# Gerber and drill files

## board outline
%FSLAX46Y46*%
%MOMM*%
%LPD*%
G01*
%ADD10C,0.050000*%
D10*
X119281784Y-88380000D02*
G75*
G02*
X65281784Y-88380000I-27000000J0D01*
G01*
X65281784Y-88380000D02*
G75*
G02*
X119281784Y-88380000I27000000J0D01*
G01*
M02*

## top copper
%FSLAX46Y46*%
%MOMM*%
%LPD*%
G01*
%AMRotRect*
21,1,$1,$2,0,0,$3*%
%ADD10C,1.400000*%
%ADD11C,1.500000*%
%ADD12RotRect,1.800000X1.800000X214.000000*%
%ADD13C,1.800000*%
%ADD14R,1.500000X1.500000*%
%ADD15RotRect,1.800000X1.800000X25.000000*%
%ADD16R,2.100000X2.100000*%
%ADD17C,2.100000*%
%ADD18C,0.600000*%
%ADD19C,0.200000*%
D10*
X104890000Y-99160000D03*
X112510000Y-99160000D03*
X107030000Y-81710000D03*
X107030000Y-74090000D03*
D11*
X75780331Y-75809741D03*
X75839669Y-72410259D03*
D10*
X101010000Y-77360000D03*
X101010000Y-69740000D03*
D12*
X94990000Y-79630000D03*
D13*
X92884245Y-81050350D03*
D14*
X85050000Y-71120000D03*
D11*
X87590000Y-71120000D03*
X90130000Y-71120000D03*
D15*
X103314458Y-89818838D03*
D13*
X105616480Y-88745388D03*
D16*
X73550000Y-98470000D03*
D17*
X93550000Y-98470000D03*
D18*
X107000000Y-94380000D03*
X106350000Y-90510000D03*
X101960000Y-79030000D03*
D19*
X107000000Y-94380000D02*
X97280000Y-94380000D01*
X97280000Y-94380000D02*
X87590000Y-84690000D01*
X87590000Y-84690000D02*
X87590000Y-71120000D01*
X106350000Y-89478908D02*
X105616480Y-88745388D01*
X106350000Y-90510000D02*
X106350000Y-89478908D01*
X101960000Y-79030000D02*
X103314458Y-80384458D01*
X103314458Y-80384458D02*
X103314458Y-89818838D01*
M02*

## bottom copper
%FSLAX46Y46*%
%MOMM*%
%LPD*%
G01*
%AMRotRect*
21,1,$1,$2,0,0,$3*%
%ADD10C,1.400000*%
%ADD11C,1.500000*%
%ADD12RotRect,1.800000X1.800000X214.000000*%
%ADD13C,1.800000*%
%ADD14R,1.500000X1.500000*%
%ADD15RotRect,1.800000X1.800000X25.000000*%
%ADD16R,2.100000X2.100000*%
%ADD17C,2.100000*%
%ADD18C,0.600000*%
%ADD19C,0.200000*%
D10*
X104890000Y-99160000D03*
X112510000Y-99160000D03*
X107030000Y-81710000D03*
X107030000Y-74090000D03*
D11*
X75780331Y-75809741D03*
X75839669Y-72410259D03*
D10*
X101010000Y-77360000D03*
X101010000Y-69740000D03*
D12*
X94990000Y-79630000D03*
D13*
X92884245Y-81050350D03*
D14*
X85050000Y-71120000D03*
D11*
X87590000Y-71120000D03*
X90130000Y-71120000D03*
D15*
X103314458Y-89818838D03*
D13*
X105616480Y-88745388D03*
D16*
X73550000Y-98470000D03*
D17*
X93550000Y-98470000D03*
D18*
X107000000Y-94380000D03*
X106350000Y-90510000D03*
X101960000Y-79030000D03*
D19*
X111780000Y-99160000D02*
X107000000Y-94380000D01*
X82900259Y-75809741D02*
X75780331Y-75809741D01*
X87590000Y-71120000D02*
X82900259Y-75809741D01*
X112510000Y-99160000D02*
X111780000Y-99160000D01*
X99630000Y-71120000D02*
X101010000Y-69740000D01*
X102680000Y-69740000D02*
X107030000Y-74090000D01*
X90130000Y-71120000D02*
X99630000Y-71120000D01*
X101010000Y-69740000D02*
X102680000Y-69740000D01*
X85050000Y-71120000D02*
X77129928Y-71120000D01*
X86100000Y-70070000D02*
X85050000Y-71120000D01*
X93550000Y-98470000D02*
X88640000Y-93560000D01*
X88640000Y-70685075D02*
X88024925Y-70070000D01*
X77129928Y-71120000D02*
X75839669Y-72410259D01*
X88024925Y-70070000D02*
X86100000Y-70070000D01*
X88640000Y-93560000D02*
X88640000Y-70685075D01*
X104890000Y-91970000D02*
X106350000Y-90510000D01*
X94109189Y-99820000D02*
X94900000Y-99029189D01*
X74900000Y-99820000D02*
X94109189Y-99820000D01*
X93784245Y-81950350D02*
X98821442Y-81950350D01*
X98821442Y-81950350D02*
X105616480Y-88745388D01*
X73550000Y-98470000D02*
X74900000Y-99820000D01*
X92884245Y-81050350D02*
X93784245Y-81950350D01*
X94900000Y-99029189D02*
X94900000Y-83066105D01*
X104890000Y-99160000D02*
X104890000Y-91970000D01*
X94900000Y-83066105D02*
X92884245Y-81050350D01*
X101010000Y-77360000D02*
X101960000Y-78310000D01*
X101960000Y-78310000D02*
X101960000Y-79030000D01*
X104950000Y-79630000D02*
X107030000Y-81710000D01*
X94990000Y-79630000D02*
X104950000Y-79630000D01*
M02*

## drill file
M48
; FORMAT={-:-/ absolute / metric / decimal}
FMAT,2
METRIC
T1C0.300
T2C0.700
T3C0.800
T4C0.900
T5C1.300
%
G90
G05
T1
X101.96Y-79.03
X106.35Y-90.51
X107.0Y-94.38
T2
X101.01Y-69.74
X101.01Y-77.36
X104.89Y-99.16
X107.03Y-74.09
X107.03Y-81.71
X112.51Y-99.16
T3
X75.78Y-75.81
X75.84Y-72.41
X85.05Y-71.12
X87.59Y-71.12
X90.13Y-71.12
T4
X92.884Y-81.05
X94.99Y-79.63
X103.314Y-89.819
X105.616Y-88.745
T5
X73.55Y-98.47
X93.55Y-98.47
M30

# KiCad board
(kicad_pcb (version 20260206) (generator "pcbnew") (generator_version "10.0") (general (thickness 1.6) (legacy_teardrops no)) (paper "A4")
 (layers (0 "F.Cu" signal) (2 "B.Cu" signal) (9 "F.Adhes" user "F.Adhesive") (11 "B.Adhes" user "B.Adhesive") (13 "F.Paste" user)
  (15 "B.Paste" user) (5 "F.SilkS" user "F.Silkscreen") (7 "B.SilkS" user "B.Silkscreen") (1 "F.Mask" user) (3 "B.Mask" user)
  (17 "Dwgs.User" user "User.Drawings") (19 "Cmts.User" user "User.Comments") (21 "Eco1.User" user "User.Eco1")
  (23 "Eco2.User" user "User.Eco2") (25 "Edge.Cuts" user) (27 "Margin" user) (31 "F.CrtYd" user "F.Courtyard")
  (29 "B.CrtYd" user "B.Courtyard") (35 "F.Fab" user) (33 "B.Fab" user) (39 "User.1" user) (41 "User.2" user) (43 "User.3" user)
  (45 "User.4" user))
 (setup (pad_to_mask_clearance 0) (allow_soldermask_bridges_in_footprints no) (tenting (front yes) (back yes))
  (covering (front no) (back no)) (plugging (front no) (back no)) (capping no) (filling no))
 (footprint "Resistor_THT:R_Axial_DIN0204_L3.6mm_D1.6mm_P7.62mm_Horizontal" (layer "F.Cu") (at 104.89 99.16)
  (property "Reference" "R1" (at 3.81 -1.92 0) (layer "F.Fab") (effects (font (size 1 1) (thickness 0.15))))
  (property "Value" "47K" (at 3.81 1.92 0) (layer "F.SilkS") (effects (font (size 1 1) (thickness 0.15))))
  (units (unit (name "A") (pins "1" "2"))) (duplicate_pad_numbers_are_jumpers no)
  (pad "1" thru_hole circle (at 0 0) (size 1.4 1.4) (drill 0.7) (layers "*.Cu" "*.Mask") (remove_unused_layers no) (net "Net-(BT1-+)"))
  (pad "2" thru_hole circle (at 7.62 0) (size 1.4 1.4) (drill 0.7) (layers "*.Cu" "*.Mask") (remove_unused_layers no) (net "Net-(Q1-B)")))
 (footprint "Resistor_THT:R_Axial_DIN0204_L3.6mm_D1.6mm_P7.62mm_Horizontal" (layer "F.Cu") (at 107.03 81.71 90)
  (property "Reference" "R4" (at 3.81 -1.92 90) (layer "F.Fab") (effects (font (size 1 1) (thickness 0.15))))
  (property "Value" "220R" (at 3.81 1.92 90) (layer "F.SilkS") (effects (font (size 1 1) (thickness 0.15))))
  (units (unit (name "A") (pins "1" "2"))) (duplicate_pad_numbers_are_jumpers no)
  (pad "1" thru_hole circle (at 0 0 90) (size 1.4 1.4) (drill 0.7) (layers "*.Cu" "*.Mask") (remove_unused_layers no) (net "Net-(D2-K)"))
  (pad "2" thru_hole circle (at 7.62 0 90) (size 1.4 1.4) (drill 0.7) (layers "*.Cu" "*.Mask") (remove_unused_layers no) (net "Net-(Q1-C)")))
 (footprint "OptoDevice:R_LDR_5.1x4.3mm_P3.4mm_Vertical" (layer "F.Cu") (at 75.780331 75.809741 89)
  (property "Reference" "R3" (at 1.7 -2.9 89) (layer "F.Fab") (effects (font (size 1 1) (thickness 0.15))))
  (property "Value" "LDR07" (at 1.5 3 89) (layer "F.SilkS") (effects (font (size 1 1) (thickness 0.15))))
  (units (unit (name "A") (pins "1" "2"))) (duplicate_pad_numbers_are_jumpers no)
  (pad "1" thru_hole circle (at 0 0 89) (size 1.5 1.5) (drill 0.8) (layers "*.Cu" "*.Mask") (remove_unused_layers no) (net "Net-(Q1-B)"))
  (pad "2" thru_hole circle (at 3.4 0 89) (size 1.5 1.5) (drill 0.8) (layers "*.Cu" "*.Mask") (remove_unused_layers no) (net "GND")))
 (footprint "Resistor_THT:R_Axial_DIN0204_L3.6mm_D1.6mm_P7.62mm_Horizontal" (layer "F.Cu") (at 101.01 77.36 90)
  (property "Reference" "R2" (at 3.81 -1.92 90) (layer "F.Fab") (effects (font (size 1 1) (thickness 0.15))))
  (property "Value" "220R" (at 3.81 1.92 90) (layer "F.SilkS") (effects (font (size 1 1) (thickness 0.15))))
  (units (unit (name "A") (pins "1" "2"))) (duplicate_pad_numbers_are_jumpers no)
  (pad "1" thru_hole circle (at 0 0 90) (size 1.4 1.4) (drill 0.7) (layers "*.Cu" "*.Mask") (remove_unused_layers no) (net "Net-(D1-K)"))
  (pad "2" thru_hole circle (at 7.62 0 90) (size 1.4 1.4) (drill 0.7) (layers "*.Cu" "*.Mask") (remove_unused_layers no) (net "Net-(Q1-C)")))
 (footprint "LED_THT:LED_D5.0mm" (layer "F.Cu") (at 94.99 79.63 -146)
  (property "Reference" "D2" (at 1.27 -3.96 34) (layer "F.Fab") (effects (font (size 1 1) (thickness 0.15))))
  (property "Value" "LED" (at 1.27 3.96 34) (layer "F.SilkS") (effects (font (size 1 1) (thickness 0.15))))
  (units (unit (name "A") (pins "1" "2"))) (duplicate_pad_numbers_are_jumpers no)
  (pad "1" thru_hole rect (at 0 0 214) (size 1.8 1.8) (drill 0.9) (layers "*.Cu" "*.Mask") (remove_unused_layers no) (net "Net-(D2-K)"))
  (pad "2" thru_hole circle (at 2.54 0 214) (size 1.8 1.8) (drill 0.9) (layers "*.Cu" "*.Mask") (remove_unused_layers no)
   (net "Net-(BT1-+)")))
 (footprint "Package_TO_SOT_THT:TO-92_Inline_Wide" (layer "F.Cu") (at 85.05 71.12)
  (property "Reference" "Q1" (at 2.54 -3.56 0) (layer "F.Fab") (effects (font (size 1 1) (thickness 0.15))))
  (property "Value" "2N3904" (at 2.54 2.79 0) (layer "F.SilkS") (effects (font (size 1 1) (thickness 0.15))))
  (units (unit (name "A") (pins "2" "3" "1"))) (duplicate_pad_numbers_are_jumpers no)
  (pad "1" thru_hole rect (at 0 0) (size 1.5 1.5) (drill 0.8) (layers "*.Cu" "*.Mask") (remove_unused_layers no) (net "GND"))
  (pad "2" thru_hole circle (at 2.54 0) (size 1.5 1.5) (drill 0.8) (layers "*.Cu" "*.Mask") (remove_unused_layers no) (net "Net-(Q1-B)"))
  (pad "3" thru_hole circle (at 5.08 0) (size 1.5 1.5) (drill 0.8) (layers "*.Cu" "*.Mask") (remove_unused_layers no) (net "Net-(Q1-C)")))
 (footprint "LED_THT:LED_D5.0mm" (layer "F.Cu") (at 103.314458 89.818838 25)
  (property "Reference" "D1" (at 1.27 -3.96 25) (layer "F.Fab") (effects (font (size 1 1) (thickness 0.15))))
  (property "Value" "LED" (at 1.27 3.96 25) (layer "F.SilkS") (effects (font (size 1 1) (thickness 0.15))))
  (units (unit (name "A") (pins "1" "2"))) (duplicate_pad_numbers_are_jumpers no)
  (pad "1" thru_hole rect (at 0 0 25) (size 1.8 1.8) (drill 0.9) (layers "*.Cu" "*.Mask") (remove_unused_layers no) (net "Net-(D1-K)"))
  (pad "2" thru_hole circle (at 2.54 0 25) (size 1.8 1.8) (drill 0.9) (layers "*.Cu" "*.Mask") (remove_unused_layers no) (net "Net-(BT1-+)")))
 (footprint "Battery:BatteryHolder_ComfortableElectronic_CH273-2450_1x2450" (layer "B.Cu") (at 73.55 98.47)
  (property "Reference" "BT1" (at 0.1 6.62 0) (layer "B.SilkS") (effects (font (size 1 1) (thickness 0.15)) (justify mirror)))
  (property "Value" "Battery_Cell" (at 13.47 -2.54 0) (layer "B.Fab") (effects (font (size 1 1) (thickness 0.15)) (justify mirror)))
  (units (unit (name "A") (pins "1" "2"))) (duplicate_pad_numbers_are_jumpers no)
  (pad "1" thru_hole rect (at 0 0 90) (size 2.1 2.1) (drill 1.3) (layers "*.Cu" "*.Mask") (remove_unused_layers no) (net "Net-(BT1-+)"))
  (pad "2" thru_hole circle (at 20 0 90) (size 2.1 2.1) (drill 1.3) (layers "*.Cu" "*.Mask") (remove_unused_layers no) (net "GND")))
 (gr_circle (center 92.281784 88.38) (end 119.281784 88.38) (stroke (width 0.05) (type solid)) (fill no) (layer "Edge.Cuts"))
 (segment (start 107 94.38) (end 97.28 94.38) (width 0.2) (layer "F.Cu") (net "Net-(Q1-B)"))
 (segment (start 97.28 94.38) (end 87.59 84.69) (width 0.2) (layer "F.Cu") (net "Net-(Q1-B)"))
 (segment (start 87.59 84.69) (end 87.59 71.12) (width 0.2) (layer "F.Cu") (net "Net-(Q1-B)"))
 (via (at 107 94.38) (size 0.6) (drill 0.3) (layers "F.Cu" "B.Cu") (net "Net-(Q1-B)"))
 (segment (start 111.78 99.16) (end 107 94.38) (width 0.2) (layer "B.Cu") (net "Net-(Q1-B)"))
 (segment (start 82.900259 75.809741) (end 75.780331 75.809741) (width 0.2) (layer "B.Cu") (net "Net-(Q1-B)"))
 (segment (start 87.59 71.12) (end 82.900259 75.809741) (width 0.2) (layer "B.Cu") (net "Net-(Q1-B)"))
 (segment (start 112.51 99.16) (end 111.78 99.16) (width 0.2) (layer "B.Cu") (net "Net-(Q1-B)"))
 (segment (start 99.63 71.12) (end 101.01 69.74) (width 0.2) (layer "B.Cu") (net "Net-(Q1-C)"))
 (segment (start 102.68 69.74) (end 107.03 74.09) (width 0.2) (layer "B.Cu") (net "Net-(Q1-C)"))
 (segment (start 90.13 71.12) (end 99.63 71.12) (width 0.2) (layer "B.Cu") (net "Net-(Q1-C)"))
 (segment (start 101.01 69.74) (end 102.68 69.74) (width 0.2) (layer "B.Cu") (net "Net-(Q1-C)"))
 (segment (start 85.05 71.12) (end 77.129928 71.12) (width 0.2) (layer "B.Cu") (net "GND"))
 (segment (start 86.1 70.07) (end 85.05 71.12) (width 0.2) (layer "B.Cu") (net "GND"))
 (segment (start 93.55 98.47) (end 88.64 93.56) (width 0.2) (layer "B.Cu") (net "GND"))
 (segment (start 88.64 70.685075) (end 88.024925 70.07) (width 0.2) (layer "B.Cu") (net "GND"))
 (segment (start 77.129928 71.12) (end 75.839669 72.410259) (width 0.2) (layer "B.Cu") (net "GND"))
 (segment (start 88.024925 70.07) (end 86.1 70.07) (width 0.2) (layer "B.Cu") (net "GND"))
 (segment (start 88.64 93.56) (end 88.64 70.685075) (width 0.2) (layer "B.Cu") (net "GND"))
 (segment (start 106.35 89.478908) (end 105.61648 88.745388) (width 0.2) (layer "F.Cu") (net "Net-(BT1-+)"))
 (segment (start 106.35 90.51) (end 106.35 89.478908) (width 0.2) (layer "F.Cu") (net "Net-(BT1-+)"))
 (via (at 106.35 90.51) (size 0.6) (drill 0.3) (layers "F.Cu" "B.Cu") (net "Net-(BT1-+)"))
 (segment (start 104.89 91.97) (end 106.35 90.51) (width 0.2) (layer "B.Cu") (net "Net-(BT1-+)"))
 (segment (start 94.109189 99.82) (end 94.9 99.029189) (width 0.2) (layer "B.Cu") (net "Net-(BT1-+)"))
 (segment (start 74.9 99.82) (end 94.109189 99.82) (width 0.2) (layer "B.Cu") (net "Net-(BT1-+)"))
 (segment (start 93.784245 81.95035) (end 98.821442 81.95035) (width 0.2) (layer "B.Cu") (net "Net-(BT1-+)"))
 (segment (start 98.821442 81.95035) (end 105.61648 88.745388) (width 0.2) (layer "B.Cu") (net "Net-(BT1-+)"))
 (segment (start 73.55 98.47) (end 74.9 99.82) (width 0.2) (layer "B.Cu") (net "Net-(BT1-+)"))
 (segment (start 92.884245 81.05035) (end 93.784245 81.95035) (width 0.2) (layer "B.Cu") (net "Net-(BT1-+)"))
 (segment (start 94.9 99.029189) (end 94.9 83.066105) (width 0.2) (layer "B.Cu") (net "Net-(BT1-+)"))
 (segment (start 104.89 99.16) (end 104.89 91.97) (width 0.2) (layer "B.Cu") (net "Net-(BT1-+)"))
 (segment (start 94.9 83.066105) (end 92.884245 81.05035) (width 0.2) (layer "B.Cu") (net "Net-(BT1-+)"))
 (segment (start 101.96 79.03) (end 103.314458 80.384458) (width 0.2) (layer "F.Cu") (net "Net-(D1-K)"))
 (segment (start 103.314458 80.384458) (end 103.314458 89.818838) (width 0.2) (layer "F.Cu") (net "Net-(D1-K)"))
 (via (at 101.96 79.03) (size 0.6) (drill 0.3) (layers "F.Cu" "B.Cu") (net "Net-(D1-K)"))
 (segment (start 101.01 77.36) (end 101.96 78.31) (width 0.2) (layer "B.Cu") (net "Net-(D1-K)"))
 (segment (start 101.96 78.31) (end 101.96 79.03) (width 0.2) (layer "B.Cu") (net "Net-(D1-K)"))
 (segment (start 104.95 79.63) (end 107.03 81.71) (width 0.2) (layer "B.Cu") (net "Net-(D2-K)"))
 (segment (start 94.99 79.63) (end 104.95 79.63) (width 0.2) (layer "B.Cu") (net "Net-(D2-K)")))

